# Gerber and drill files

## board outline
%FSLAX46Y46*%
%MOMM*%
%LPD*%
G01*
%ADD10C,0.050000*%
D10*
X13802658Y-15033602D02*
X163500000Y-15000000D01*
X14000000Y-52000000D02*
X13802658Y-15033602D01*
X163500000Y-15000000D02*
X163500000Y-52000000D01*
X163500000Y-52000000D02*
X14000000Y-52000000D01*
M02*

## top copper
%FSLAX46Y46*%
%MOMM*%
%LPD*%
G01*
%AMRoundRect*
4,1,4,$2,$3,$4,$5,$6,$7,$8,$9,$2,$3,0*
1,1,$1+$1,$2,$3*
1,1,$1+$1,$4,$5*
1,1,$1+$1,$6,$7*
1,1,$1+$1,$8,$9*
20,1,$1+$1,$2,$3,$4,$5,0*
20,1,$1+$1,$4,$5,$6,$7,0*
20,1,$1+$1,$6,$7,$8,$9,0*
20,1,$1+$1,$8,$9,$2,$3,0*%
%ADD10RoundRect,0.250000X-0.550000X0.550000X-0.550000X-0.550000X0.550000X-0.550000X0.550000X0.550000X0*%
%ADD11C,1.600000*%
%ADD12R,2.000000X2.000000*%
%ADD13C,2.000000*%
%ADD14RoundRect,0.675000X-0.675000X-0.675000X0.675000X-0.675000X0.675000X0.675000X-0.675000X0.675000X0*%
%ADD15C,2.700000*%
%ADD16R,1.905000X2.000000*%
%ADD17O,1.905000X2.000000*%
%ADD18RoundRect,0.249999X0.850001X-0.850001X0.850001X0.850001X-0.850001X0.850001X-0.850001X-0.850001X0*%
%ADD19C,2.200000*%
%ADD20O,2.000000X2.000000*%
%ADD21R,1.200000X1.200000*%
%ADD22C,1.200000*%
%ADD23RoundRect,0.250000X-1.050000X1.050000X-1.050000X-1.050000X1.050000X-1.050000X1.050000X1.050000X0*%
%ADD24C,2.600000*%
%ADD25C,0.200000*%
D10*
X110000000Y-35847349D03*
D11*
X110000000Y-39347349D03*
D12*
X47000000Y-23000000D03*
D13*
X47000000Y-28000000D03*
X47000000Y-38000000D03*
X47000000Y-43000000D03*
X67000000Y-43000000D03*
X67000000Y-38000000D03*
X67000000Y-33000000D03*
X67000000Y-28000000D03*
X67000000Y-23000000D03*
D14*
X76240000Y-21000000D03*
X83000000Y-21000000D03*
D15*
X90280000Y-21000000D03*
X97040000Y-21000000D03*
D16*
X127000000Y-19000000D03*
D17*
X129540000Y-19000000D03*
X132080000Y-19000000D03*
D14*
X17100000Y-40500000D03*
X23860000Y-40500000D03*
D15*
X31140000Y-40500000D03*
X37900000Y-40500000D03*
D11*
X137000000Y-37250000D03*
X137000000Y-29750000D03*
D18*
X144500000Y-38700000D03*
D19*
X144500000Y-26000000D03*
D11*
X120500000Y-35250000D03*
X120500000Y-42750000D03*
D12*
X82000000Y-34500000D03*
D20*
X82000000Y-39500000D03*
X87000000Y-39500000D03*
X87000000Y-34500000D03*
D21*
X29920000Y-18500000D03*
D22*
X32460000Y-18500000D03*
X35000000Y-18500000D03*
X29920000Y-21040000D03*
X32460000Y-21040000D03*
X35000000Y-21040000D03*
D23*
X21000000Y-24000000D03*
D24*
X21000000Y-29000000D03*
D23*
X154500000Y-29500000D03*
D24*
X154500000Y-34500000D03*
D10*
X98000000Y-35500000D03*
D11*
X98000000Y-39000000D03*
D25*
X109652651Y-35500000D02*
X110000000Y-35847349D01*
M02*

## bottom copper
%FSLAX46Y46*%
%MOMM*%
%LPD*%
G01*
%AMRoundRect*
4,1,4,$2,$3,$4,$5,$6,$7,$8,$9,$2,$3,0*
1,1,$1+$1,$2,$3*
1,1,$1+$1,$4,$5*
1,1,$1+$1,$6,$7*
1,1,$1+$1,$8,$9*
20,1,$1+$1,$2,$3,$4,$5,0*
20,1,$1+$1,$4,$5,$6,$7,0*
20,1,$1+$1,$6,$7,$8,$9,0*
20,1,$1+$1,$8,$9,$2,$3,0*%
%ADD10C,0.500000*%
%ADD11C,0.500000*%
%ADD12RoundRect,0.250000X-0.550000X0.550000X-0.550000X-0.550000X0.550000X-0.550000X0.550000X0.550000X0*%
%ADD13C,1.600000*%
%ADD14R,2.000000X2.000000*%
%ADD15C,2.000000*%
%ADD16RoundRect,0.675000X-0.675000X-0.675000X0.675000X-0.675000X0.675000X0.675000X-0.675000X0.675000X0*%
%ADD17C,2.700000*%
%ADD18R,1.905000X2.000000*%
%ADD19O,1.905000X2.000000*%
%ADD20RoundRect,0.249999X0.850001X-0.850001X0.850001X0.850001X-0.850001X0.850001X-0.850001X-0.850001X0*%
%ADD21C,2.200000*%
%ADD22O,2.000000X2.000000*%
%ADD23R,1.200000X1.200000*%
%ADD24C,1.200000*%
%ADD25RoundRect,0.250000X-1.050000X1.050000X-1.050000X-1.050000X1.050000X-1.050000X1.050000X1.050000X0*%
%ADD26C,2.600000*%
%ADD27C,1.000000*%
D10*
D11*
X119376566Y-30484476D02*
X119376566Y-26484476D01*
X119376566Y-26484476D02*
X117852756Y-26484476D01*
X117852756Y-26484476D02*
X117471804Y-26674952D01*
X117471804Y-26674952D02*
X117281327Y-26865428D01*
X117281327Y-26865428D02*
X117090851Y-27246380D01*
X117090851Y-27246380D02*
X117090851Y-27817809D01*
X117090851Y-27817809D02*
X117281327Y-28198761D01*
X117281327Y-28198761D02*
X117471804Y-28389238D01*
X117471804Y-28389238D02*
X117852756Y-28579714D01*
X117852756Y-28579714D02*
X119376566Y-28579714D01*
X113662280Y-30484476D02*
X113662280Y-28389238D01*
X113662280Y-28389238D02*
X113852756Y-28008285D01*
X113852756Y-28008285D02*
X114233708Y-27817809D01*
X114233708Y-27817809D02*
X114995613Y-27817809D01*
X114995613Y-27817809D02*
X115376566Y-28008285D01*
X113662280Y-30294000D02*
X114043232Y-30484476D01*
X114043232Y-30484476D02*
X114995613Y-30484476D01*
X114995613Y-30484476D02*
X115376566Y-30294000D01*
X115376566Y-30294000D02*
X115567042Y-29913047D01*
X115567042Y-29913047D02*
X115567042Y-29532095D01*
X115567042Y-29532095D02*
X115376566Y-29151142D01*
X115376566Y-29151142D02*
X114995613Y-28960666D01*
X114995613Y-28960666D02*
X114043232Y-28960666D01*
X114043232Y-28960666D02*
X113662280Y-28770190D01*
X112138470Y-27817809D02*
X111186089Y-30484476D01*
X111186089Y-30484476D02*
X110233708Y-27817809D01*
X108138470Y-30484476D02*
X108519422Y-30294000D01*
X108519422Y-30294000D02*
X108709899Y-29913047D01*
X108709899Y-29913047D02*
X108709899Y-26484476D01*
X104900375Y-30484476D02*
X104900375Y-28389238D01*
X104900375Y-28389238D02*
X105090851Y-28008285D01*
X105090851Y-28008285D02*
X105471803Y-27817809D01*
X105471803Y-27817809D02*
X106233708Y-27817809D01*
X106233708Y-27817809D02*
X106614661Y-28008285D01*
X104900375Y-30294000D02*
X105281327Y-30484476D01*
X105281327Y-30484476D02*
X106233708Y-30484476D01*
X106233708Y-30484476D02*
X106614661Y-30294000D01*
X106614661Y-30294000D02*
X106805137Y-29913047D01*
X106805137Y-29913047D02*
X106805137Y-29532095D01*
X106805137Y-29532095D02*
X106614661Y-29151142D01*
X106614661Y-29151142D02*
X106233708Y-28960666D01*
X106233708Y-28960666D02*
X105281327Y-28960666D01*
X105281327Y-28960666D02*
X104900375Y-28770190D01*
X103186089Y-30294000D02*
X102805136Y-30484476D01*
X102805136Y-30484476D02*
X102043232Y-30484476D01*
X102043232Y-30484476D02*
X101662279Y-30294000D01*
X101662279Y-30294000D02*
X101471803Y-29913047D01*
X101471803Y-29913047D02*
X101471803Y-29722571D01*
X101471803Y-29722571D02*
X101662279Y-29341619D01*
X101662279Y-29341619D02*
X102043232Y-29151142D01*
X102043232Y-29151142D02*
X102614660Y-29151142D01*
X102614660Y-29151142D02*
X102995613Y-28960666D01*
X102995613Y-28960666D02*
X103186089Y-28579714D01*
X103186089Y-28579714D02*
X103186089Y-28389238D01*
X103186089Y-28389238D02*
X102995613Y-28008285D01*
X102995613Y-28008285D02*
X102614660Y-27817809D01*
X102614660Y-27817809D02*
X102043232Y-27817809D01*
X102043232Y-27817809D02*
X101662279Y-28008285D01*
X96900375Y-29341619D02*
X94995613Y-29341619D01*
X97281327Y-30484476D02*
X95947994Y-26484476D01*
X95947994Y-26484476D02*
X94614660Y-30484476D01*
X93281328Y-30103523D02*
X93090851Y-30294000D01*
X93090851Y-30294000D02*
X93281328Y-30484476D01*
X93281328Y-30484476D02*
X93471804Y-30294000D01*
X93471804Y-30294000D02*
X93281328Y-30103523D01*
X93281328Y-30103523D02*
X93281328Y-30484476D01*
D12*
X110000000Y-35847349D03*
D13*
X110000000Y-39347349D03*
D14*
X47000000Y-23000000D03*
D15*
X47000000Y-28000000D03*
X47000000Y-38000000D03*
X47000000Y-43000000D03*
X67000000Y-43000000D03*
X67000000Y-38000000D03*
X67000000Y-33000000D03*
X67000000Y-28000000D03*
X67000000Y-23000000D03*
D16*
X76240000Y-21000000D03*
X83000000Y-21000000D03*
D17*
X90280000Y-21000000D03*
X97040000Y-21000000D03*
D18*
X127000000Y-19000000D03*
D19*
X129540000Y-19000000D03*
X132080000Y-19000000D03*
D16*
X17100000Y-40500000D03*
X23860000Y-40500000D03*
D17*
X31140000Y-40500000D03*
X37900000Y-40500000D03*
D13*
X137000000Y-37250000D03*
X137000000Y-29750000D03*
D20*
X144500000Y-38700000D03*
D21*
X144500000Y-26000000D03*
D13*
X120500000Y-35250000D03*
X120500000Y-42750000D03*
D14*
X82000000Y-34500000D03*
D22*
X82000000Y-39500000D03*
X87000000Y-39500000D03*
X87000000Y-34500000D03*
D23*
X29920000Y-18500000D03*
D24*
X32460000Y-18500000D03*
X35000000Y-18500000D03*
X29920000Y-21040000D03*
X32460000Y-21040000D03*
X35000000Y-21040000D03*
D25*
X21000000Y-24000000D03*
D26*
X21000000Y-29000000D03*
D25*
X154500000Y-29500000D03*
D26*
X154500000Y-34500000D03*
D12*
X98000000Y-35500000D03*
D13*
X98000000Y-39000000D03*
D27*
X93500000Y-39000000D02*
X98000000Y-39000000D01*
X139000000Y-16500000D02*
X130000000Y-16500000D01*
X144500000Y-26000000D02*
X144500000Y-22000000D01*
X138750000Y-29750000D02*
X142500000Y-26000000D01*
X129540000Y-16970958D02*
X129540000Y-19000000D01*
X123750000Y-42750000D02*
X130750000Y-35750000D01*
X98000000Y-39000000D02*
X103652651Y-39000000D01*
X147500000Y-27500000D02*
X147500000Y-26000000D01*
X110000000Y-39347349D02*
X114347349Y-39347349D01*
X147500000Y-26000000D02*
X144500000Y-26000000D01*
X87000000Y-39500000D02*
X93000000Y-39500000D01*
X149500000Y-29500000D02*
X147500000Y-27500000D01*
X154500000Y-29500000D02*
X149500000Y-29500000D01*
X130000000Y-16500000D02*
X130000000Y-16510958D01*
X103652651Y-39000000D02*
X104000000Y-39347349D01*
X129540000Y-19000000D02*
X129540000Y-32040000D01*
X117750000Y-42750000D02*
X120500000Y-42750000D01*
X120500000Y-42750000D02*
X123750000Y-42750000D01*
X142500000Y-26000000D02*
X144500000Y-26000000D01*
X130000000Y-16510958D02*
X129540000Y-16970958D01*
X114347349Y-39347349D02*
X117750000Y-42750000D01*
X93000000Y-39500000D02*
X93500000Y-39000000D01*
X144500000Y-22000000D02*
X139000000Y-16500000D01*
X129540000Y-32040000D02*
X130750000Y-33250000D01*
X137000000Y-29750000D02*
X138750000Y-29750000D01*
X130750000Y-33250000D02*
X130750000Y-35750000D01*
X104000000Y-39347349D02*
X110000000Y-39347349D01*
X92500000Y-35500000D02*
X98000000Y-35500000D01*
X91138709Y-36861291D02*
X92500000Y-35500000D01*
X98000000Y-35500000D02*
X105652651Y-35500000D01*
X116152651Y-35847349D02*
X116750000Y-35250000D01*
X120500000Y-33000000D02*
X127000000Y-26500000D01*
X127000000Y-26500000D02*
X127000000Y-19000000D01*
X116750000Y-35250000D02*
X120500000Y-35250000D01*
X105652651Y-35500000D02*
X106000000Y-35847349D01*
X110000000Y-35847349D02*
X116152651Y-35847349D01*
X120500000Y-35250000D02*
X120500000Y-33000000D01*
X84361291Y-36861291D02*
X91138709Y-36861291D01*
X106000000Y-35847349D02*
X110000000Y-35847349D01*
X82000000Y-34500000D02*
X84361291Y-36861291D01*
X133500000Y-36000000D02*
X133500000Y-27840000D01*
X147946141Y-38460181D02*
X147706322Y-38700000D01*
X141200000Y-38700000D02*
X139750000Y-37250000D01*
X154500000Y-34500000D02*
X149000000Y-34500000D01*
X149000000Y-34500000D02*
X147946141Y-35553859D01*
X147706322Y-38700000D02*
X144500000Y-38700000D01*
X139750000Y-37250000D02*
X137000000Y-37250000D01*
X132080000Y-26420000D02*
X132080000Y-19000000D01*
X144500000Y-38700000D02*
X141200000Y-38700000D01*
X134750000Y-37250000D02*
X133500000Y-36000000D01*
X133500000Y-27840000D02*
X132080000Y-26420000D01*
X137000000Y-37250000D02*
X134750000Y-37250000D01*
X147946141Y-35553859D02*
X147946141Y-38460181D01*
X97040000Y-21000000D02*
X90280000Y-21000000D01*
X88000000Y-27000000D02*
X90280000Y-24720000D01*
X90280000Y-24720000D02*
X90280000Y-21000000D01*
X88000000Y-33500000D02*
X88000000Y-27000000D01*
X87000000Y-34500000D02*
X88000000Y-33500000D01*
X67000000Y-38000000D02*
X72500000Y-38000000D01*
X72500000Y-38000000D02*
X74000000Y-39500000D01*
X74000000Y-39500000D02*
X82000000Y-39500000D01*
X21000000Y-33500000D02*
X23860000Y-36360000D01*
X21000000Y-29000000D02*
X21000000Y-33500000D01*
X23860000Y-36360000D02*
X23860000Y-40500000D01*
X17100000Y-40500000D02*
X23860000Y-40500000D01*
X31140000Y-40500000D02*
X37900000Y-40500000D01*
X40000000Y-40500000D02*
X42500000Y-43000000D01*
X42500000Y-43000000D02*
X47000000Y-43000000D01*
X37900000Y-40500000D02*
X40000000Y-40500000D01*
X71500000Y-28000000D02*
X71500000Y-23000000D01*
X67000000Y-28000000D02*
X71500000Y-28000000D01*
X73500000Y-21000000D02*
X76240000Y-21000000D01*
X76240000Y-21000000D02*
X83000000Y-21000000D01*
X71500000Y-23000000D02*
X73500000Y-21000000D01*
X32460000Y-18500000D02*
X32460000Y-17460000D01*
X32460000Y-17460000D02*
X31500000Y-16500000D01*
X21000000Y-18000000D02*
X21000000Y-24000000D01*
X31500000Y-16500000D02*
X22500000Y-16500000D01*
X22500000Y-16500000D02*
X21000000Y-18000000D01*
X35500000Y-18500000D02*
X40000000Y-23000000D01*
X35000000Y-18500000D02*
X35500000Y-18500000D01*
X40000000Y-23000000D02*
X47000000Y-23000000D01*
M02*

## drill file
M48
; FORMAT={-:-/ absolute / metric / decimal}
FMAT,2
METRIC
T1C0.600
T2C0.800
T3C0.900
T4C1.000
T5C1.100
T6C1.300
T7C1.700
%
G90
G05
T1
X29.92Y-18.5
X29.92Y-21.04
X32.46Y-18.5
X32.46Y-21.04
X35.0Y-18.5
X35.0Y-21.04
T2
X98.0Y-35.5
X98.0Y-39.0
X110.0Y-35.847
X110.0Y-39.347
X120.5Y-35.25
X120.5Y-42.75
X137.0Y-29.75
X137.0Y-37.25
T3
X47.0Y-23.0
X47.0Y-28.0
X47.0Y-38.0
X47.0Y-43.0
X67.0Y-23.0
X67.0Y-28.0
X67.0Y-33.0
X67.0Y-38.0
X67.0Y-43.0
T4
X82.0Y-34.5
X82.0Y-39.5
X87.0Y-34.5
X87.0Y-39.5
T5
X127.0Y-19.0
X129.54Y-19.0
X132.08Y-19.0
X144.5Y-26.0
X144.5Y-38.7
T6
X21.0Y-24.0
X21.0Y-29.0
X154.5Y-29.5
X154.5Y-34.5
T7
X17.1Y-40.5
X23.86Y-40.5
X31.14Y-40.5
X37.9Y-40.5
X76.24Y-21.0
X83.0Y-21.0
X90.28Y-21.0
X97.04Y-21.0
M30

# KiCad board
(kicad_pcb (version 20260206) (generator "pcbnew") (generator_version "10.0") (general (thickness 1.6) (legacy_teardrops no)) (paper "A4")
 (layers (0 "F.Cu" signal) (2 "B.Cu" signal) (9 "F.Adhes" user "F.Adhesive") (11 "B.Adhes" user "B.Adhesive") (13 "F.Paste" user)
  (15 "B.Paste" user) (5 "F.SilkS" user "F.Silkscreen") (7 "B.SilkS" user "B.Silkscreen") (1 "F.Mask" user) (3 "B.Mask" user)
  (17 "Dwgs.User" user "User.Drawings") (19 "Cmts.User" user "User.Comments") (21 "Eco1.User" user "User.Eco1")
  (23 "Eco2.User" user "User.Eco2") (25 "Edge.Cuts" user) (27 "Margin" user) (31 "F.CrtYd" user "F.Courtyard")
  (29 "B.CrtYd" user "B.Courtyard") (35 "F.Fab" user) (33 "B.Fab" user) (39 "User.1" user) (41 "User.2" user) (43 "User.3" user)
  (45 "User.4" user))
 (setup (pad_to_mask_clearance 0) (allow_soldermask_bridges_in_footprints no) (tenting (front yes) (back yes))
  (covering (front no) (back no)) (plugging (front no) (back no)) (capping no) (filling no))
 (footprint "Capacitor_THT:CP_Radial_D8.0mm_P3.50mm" (layer "F.Cu") (at 110 35.847349 -90)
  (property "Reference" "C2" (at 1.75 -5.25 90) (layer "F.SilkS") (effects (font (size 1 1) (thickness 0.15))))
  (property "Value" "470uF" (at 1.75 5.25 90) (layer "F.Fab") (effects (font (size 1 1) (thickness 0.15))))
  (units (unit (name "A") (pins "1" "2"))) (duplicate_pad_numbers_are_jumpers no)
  (pad "1" thru_hole roundrect (at 0 0 270) (size 1.6 1.6) (drill 0.8) (layers "*.Cu" "*.Mask") (remove_unused_layers no)
   (roundrect_rratio 0.15625) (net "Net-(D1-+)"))
  (pad "2" thru_hole circle (at 3.5 0 270) (size 1.6 1.6) (drill 0.8) (layers "*.Cu" "*.Mask") (remove_unused_layers no) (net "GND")))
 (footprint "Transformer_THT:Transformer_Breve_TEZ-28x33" (layer "F.Cu") (at 47 23 -90)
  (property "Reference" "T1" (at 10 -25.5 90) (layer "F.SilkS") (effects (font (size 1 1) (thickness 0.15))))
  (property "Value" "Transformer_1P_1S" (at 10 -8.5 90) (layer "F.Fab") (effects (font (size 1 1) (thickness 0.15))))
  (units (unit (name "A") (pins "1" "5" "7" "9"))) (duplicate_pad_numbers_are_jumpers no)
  (pad "1" thru_hole rect (at 0 0 270) (size 2 2) (drill 0.9) (layers "*.Cu" "*.Mask") (remove_unused_layers no) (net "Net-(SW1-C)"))
  (pad "2" thru_hole circle (at 5 0 270) (size 2 2) (drill 0.9) (layers "*.Cu" "*.Mask") (remove_unused_layers no))
  (pad "4" thru_hole circle (at 15 0 270) (size 2 2) (drill 0.9) (layers "*.Cu" "*.Mask") (remove_unused_layers no))
  (pad "5" thru_hole circle (at 20 0 270) (size 2 2) (drill 0.9) (layers "*.Cu" "*.Mask") (remove_unused_layers no) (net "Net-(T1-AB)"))
  (pad "6" thru_hole circle (at 20 -20 270) (size 2 2) (drill 0.9) (layers "*.Cu" "*.Mask") (remove_unused_layers no))
  (pad "7" thru_hole circle (at 15 -20 270) (size 2 2) (drill 0.9) (layers "*.Cu" "*.Mask") (remove_unused_layers no) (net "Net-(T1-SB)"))
  (pad "8" thru_hole circle (at 10 -20 270) (size 2 2) (drill 0.9) (layers "*.Cu" "*.Mask") (remove_unused_layers no))
  (pad "9" thru_hole circle (at 5 -20 270) (size 2 2) (drill 0.9) (layers "*.Cu" "*.Mask") (remove_unused_layers no) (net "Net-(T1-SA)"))
  (pad "10" thru_hole circle (at 0 -20 270) (size 2 2) (drill 0.9) (layers "*.Cu" "*.Mask") (remove_unused_layers no)))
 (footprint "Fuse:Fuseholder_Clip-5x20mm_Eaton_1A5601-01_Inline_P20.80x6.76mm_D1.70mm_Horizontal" (layer "F.Cu") (at 76.24 21)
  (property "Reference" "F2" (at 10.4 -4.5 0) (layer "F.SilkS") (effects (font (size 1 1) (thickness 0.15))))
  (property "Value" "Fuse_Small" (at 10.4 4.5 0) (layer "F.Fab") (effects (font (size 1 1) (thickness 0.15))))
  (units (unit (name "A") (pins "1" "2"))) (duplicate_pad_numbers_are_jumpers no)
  (pad "1" thru_hole roundrect (at 0 0) (size 2.7 2.7) (drill 1.7) (layers "*.Cu" "*.Mask") (remove_unused_layers no)
   (roundrect_rratio 0.25) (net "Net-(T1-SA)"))
  (pad "1" thru_hole roundrect (at 6.76 0) (size 2.7 2.7) (drill 1.7) (layers "*.Cu" "*.Mask") (remove_unused_layers no)
   (roundrect_rratio 0.25) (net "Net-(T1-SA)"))
  (pad "2" thru_hole circle (at 14.04 0) (size 2.7 2.7) (drill 1.7) (layers "*.Cu" "*.Mask") (remove_unused_layers no) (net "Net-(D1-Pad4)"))
  (pad "2" thru_hole circle (at 20.8 0) (size 2.7 2.7) (drill 1.7) (layers "*.Cu" "*.Mask") (remove_unused_layers no) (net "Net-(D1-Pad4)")))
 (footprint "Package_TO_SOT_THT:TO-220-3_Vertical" (layer "F.Cu") (at 127 19)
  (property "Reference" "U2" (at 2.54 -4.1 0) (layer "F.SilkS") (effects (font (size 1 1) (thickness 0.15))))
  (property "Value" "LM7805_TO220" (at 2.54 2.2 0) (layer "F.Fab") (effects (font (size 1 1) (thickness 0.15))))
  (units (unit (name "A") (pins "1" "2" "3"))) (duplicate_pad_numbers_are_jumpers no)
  (pad "1" thru_hole rect (at 0 0) (size 1.905 2) (drill 1.1) (layers "*.Cu" "*.Mask") (remove_unused_layers no) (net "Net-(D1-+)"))
  (pad "2" thru_hole oval (at 2.54 0) (size 1.905 2) (drill 1.1) (layers "*.Cu" "*.Mask") (remove_unused_layers no) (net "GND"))
  (pad "3" thru_hole oval (at 5.08 0) (size 1.905 2) (drill 1.1) (layers "*.Cu" "*.Mask") (remove_unused_layers no) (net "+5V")))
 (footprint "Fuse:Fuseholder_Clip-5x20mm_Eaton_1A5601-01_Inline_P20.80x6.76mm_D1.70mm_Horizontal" (layer "F.Cu") (at 17.1 40.5)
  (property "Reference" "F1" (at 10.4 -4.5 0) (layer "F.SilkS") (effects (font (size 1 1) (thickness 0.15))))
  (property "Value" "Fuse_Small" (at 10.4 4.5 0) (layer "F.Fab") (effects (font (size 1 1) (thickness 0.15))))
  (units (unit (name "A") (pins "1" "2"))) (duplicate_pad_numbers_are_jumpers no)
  (pad "1" thru_hole roundrect (at 0 0) (size 2.7 2.7) (drill 1.7) (layers "*.Cu" "*.Mask") (remove_unused_layers no)
   (roundrect_rratio 0.25) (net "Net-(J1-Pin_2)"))
  (pad "1" thru_hole roundrect (at 6.76 0) (size 2.7 2.7) (drill 1.7) (layers "*.Cu" "*.Mask") (remove_unused_layers no)
   (roundrect_rratio 0.25) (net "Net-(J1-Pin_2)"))
  (pad "2" thru_hole circle (at 14.04 0) (size 2.7 2.7) (drill 1.7) (layers "*.Cu" "*.Mask") (remove_unused_layers no) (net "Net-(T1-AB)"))
  (pad "2" thru_hole circle (at 20.8 0) (size 2.7 2.7) (drill 1.7) (layers "*.Cu" "*.Mask") (remove_unused_layers no) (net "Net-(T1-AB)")))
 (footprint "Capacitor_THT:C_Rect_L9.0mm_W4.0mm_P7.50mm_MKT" (layer "F.Cu") (at 137 37.25 90)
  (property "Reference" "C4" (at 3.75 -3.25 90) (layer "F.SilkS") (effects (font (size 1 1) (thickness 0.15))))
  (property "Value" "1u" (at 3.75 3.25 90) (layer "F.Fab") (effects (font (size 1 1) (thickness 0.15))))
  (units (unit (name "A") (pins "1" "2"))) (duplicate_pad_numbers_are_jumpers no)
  (pad "1" thru_hole circle (at 0 0 90) (size 1.6 1.6) (drill 0.8) (layers "*.Cu" "*.Mask") (remove_unused_layers no) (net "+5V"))
  (pad "2" thru_hole circle (at 7.5 0 90) (size 1.6 1.6) (drill 0.8) (layers "*.Cu" "*.Mask") (remove_unused_layers no) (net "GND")))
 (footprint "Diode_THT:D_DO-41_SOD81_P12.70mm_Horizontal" (layer "F.Cu") (at 144.5 38.7 90)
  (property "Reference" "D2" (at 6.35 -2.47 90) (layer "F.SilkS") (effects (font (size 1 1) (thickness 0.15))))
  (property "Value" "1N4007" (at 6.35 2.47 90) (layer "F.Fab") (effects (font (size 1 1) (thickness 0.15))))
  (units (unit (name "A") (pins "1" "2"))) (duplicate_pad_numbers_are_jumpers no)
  (pad "1" thru_hole roundrect (at 0 0 90) (size 2.2 2.2) (drill 1.1) (layers "*.Cu" "*.Mask") (remove_unused_layers no)
   (roundrect_rratio 0.113636) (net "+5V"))
  (pad "2" thru_hole circle (at 12.7 0 90) (size 2.2 2.2) (drill 1.1) (layers "*.Cu" "*.Mask") (remove_unused_layers no) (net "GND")))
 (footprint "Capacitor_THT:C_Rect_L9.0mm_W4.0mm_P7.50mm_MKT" (layer "F.Cu") (at 120.5 35.25 -90)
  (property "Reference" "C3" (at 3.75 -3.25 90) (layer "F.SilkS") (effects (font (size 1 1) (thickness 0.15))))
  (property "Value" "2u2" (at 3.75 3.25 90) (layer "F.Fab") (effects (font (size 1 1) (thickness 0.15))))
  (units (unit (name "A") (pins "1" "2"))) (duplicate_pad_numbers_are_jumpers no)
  (pad "1" thru_hole circle (at 0 0 270) (size 1.6 1.6) (drill 0.8) (layers "*.Cu" "*.Mask") (remove_unused_layers no) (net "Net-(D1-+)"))
  (pad "2" thru_hole circle (at 7.5 0 270) (size 1.6 1.6) (drill 0.8) (layers "*.Cu" "*.Mask") (remove_unused_layers no) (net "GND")))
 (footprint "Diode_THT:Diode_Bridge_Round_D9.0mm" (layer "F.Cu") (at 82 34.5)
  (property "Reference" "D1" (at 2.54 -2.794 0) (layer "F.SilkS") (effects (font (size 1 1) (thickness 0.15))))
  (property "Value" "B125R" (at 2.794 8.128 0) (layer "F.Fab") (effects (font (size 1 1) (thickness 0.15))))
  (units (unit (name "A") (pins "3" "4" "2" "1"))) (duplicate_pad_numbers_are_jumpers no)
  (pad "1" thru_hole rect (at 0 0) (size 2 2) (drill 1) (layers "*.Cu" "*.Mask") (remove_unused_layers no) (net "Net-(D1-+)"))
  (pad "2" thru_hole oval (at 0 5) (size 2 2) (drill 1) (layers "*.Cu" "*.Mask") (remove_unused_layers no) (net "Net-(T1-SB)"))
  (pad "3" thru_hole oval (at 5 5) (size 2 2) (drill 1) (layers "*.Cu" "*.Mask") (remove_unused_layers no) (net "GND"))
  (pad "4" thru_hole oval (at 5 0) (size 2 2) (drill 1) (layers "*.Cu" "*.Mask") (remove_unused_layers no) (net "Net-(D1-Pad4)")))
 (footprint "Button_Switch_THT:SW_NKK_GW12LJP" (layer "F.Cu") (at 29.92 18.5)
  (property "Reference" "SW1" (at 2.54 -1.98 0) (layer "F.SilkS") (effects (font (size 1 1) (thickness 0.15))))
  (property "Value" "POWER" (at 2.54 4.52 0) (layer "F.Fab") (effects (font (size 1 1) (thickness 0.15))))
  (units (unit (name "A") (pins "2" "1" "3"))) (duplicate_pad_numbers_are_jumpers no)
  (pad "1" thru_hole rect (at 0 0) (size 1.2 1.2) (drill 0.6) (layers "*.Cu" "*.Mask") (remove_unused_layers no)
   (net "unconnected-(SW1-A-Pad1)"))
  (pad "2" thru_hole circle (at 2.54 0) (size 1.2 1.2) (drill 0.6) (layers "*.Cu" "*.Mask") (remove_unused_layers no) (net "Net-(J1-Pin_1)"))
  (pad "3" thru_hole circle (at 5.08 0) (size 1.2 1.2) (drill 0.6) (layers "*.Cu" "*.Mask") (remove_unused_layers no) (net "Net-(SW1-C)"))
  (pad "4" thru_hole circle (at 0 2.54) (size 1.2 1.2) (drill 0.6) (layers "*.Cu" "*.Mask") (remove_unused_layers no))
  (pad "5" thru_hole circle (at 2.54 2.54) (size 1.2 1.2) (drill 0.6) (layers "*.Cu" "*.Mask") (remove_unused_layers no))
  (pad "6" thru_hole circle (at 5.08 2.54) (size 1.2 1.2) (drill 0.6) (layers "*.Cu" "*.Mask") (remove_unused_layers no)))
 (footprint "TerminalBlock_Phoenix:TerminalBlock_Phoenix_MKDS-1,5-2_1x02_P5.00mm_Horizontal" (layer "F.Cu") (at 21 24 -90)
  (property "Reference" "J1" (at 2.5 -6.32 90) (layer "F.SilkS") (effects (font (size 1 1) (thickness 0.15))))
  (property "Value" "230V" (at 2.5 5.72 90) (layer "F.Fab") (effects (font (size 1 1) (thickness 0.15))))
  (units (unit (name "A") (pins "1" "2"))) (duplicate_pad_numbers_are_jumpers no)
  (pad "1" thru_hole roundrect (at 0 0 270) (size 2.6 2.6) (drill 1.3) (layers "*.Cu" "*.Mask") (remove_unused_layers no)
   (roundrect_rratio 0.096154) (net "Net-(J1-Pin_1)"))
  (pad "2" thru_hole circle (at 5 0 270) (size 2.6 2.6) (drill 1.3) (layers "*.Cu" "*.Mask") (remove_unused_layers no)
   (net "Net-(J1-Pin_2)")))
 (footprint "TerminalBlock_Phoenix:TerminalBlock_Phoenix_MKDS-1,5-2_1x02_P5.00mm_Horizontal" (layer "F.Cu") (at 154.5 29.5 -90)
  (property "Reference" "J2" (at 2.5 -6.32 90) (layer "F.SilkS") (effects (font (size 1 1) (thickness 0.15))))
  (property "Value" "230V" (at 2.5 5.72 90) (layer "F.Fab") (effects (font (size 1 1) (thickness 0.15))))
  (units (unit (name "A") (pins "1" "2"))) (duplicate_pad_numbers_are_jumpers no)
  (pad "1" thru_hole roundrect (at 0 0 270) (size 2.6 2.6) (drill 1.3) (layers "*.Cu" "*.Mask") (remove_unused_layers no)
   (roundrect_rratio 0.096154) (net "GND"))
  (pad "2" thru_hole circle (at 5 0 270) (size 2.6 2.6) (drill 1.3) (layers "*.Cu" "*.Mask") (remove_unused_layers no) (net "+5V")))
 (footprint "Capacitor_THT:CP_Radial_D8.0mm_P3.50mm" (layer "F.Cu") (at 98 35.5 -90)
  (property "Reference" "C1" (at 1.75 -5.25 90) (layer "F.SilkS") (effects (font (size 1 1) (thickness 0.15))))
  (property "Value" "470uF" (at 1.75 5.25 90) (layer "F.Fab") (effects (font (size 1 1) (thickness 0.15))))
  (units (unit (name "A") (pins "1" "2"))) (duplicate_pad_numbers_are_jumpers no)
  (pad "1" thru_hole roundrect (at 0 0 270) (size 1.6 1.6) (drill 0.8) (layers "*.Cu" "*.Mask") (remove_unused_layers no)
   (roundrect_rratio 0.15625) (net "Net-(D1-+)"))
  (pad "2" thru_hole circle (at 3.5 0 270) (size 1.6 1.6) (drill 0.8) (layers "*.Cu" "*.Mask") (remove_unused_layers no) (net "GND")))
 (gr_line (start 13.802658 15.033602) (end 163.5 15) (stroke (width 0.05) (type default)) (layer "Edge.Cuts"))
 (gr_line (start 14 52) (end 13.802658 15.033602) (stroke (width 0.05) (type default)) (layer "Edge.Cuts"))
 (gr_line (start 163.5 15) (end 163.5 52) (stroke (width 0.05) (type default)) (layer "Edge.Cuts"))
 (gr_line (start 163.5 52) (end 14 52) (stroke (width 0.05) (type default)) (layer "Edge.Cuts"))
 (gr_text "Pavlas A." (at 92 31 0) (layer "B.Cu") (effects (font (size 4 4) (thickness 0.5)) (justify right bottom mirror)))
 (segment (start 93.5 39) (end 98 39) (width 1) (layer "B.Cu") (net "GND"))
 (segment (start 139 16.5) (end 130 16.5) (width 1) (layer "B.Cu") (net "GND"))
 (segment (start 144.5 26) (end 144.5 22) (width 1) (layer "B.Cu") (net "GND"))
 (segment (start 138.75 29.75) (end 142.5 26) (width 1) (layer "B.Cu") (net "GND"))
 (segment (start 129.54 16.970958) (end 129.54 19) (width 1) (layer "B.Cu") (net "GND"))
 (segment (start 123.75 42.75) (end 130.75 35.75) (width 1) (layer "B.Cu") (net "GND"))
 (segment (start 98 39) (end 103.652651 39) (width 1) (layer "B.Cu") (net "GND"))
 (segment (start 147.5 27.5) (end 147.5 26) (width 1) (layer "B.Cu") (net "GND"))
 (segment (start 110 39.347349) (end 114.347349 39.347349) (width 1) (layer "B.Cu") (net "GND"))
 (segment (start 147.5 26) (end 144.5 26) (width 1) (layer "B.Cu") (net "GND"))
 (segment (start 87 39.5) (end 93 39.5) (width 1) (layer "B.Cu") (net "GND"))
 (segment (start 149.5 29.5) (end 147.5 27.5) (width 1) (layer "B.Cu") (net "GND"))
 (segment (start 154.5 29.5) (end 149.5 29.5) (width 1) (layer "B.Cu") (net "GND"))
 (segment (start 130 16.5) (end 130 16.510958) (width 1) (layer "B.Cu") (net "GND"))
 (segment (start 103.652651 39) (end 104 39.347349) (width 1) (layer "B.Cu") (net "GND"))
 (segment (start 129.54 19) (end 129.54 32.04) (width 1) (layer "B.Cu") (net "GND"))
 (segment (start 117.75 42.75) (end 120.5 42.75) (width 1) (layer "B.Cu") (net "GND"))
 (segment (start 120.5 42.75) (end 123.75 42.75) (width 1) (layer "B.Cu") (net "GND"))
 (segment (start 142.5 26) (end 144.5 26) (width 1) (layer "B.Cu") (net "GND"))
 (segment (start 130 16.510958) (end 129.54 16.970958) (width 1) (layer "B.Cu") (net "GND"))
 (segment (start 114.347349 39.347349) (end 117.75 42.75) (width 1) (layer "B.Cu") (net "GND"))
 (segment (start 93 39.5) (end 93.5 39) (width 1) (layer "B.Cu") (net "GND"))
 (segment (start 144.5 22) (end 139 16.5) (width 1) (layer "B.Cu") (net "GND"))
 (segment (start 129.54 32.04) (end 130.75 33.25) (width 1) (layer "B.Cu") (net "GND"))
 (segment (start 137 29.75) (end 138.75 29.75) (width 1) (layer "B.Cu") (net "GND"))
 (segment (start 130.75 33.25) (end 130.75 35.75) (width 1) (layer "B.Cu") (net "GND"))
 (segment (start 104 39.347349) (end 110 39.347349) (width 1) (layer "B.Cu") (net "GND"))
 (segment (start 109.652651 35.5) (end 110 35.847349) (width 0.2) (layer "F.Cu") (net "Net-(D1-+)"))
 (segment (start 92.5 35.5) (end 98 35.5) (width 1) (layer "B.Cu") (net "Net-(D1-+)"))
 (segment (start 91.138709 36.861291) (end 92.5 35.5) (width 1) (layer "B.Cu") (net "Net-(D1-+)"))
 (segment (start 98 35.5) (end 105.652651 35.5) (width 1) (layer "B.Cu") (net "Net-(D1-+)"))
 (segment (start 116.152651 35.847349) (end 116.75 35.25) (width 1) (layer "B.Cu") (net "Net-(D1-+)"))
 (segment (start 120.5 33) (end 127 26.5) (width 1) (layer "B.Cu") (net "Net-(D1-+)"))
 (segment (start 127 26.5) (end 127 19) (width 1) (layer "B.Cu") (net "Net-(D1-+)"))
 (segment (start 116.75 35.25) (end 120.5 35.25) (width 1) (layer "B.Cu") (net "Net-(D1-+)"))
 (segment (start 105.652651 35.5) (end 106 35.847349) (width 1) (layer "B.Cu") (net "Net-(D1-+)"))
 (segment (start 110 35.847349) (end 116.152651 35.847349) (width 1) (layer "B.Cu") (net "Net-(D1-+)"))
 (segment (start 120.5 35.25) (end 120.5 33) (width 1) (layer "B.Cu") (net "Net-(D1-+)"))
 (segment (start 84.361291 36.861291) (end 91.138709 36.861291) (width 1) (layer "B.Cu") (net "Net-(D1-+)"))
 (segment (start 106 35.847349) (end 110 35.847349) (width 1) (layer "B.Cu") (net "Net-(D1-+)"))
 (segment (start 82 34.5) (end 84.361291 36.861291) (width 1) (layer "B.Cu") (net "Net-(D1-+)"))
 (segment (start 133.5 36) (end 133.5 27.84) (width 1) (layer "B.Cu") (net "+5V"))
 (segment (start 147.946141 38.460181) (end 147.706322 38.7) (width 1) (layer "B.Cu") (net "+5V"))
 (segment (start 141.2 38.7) (end 139.75 37.25) (width 1) (layer "B.Cu") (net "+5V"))
 (segment (start 154.5 34.5) (end 149 34.5) (width 1) (layer "B.Cu") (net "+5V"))
 (segment (start 149 34.5) (end 147.946141 35.553859) (width 1) (layer "B.Cu") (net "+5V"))
 (segment (start 147.706322 38.7) (end 144.5 38.7) (width 1) (layer "B.Cu") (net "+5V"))
 (segment (start 139.75 37.25) (end 137 37.25) (width 1) (layer "B.Cu") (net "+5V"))
 (segment (start 132.08 26.42) (end 132.08 19) (width 1) (layer "B.Cu") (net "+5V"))
 (segment (start 144.5 38.7) (end 141.2 38.7) (width 1) (layer "B.Cu") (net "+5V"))
 (segment (start 134.75 37.25) (end 133.5 36) (width 1) (layer "B.Cu") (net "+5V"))
 (segment (start 133.5 27.84) (end 132.08 26.42) (width 1) (layer "B.Cu") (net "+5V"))
 (segment (start 137 37.25) (end 134.75 37.25) (width 1) (layer "B.Cu") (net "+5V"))
 (segment (start 147.946141 35.553859) (end 147.946141 38.460181) (width 1) (layer "B.Cu") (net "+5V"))
 (segment (start 97.04 21) (end 90.28 21) (width 1) (layer "B.Cu") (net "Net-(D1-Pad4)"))
 (segment (start 88 27) (end 90.28 24.72) (width 1) (layer "B.Cu") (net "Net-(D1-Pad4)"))
 (segment (start 90.28 24.72) (end 90.28 21) (width 1) (layer "B.Cu") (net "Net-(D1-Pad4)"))
 (segment (start 88 33.5) (end 88 27) (width 1) (layer "B.Cu") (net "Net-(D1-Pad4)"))
 (segment (start 87 34.5) (end 88 33.5) (width 1) (layer "B.Cu") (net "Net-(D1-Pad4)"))
 (segment (start 67 38) (end 72.5 38) (width 1) (layer "B.Cu") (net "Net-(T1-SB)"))
 (segment (start 72.5 38) (end 74 39.5) (width 1) (layer "B.Cu") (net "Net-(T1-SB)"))
 (segment (start 74 39.5) (end 82 39.5) (width 1) (layer "B.Cu") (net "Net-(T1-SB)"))
 (segment (start 21 33.5) (end 23.86 36.36) (width 1) (layer "B.Cu") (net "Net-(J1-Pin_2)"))
 (segment (start 21 29) (end 21 33.5) (width 1) (layer "B.Cu") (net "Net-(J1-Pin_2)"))
 (segment (start 23.86 36.36) (end 23.86 40.5) (width 1) (layer "B.Cu") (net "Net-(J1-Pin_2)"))
 (segment (start 17.1 40.5) (end 23.86 40.5) (width 1) (layer "B.Cu") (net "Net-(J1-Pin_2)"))
 (segment (start 31.14 40.5) (end 37.9 40.5) (width 1) (layer "B.Cu") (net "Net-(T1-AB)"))
 (segment (start 40 40.5) (end 42.5 43) (width 1) (layer "B.Cu") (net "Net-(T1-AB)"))
 (segment (start 42.5 43) (end 47 43) (width 1) (layer "B.Cu") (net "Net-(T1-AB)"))
 (segment (start 37.9 40.5) (end 40 40.5) (width 1) (layer "B.Cu") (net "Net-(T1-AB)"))
 (segment (start 71.5 28) (end 71.5 23) (width 1) (layer "B.Cu") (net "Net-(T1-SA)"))
 (segment (start 67 28) (end 71.5 28) (width 1) (layer "B.Cu") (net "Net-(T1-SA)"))
 (segment (start 73.5 21) (end 76.24 21) (width 1) (layer "B.Cu") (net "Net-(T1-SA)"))
 (segment (start 76.24 21) (end 83 21) (width 1) (layer "B.Cu") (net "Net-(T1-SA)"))
 (segment (start 71.5 23) (end 73.5 21) (width 1) (layer "B.Cu") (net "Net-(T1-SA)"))
 (segment (start 32.46 18.5) (end 32.46 17.46) (width 1) (layer "B.Cu") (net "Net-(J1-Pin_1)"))
 (segment (start 32.46 17.46) (end 31.5 16.5) (width 1) (layer "B.Cu") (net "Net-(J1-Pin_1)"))
 (segment (start 21 18) (end 21 24) (width 1) (layer "B.Cu") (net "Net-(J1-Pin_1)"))
 (segment (start 31.5 16.5) (end 22.5 16.5) (width 1) (layer "B.Cu") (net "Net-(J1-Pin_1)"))
 (segment (start 22.5 16.5) (end 21 18) (width 1) (layer "B.Cu") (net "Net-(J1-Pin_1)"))
 (segment (start 35.5 18.5) (end 40 23) (width 1) (layer "B.Cu") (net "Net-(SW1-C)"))
 (segment (start 35 18.5) (end 35.5 18.5) (width 1) (layer "B.Cu") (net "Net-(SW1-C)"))
 (segment (start 40 23) (end 47 23) (width 1) (layer "B.Cu") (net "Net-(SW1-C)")))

